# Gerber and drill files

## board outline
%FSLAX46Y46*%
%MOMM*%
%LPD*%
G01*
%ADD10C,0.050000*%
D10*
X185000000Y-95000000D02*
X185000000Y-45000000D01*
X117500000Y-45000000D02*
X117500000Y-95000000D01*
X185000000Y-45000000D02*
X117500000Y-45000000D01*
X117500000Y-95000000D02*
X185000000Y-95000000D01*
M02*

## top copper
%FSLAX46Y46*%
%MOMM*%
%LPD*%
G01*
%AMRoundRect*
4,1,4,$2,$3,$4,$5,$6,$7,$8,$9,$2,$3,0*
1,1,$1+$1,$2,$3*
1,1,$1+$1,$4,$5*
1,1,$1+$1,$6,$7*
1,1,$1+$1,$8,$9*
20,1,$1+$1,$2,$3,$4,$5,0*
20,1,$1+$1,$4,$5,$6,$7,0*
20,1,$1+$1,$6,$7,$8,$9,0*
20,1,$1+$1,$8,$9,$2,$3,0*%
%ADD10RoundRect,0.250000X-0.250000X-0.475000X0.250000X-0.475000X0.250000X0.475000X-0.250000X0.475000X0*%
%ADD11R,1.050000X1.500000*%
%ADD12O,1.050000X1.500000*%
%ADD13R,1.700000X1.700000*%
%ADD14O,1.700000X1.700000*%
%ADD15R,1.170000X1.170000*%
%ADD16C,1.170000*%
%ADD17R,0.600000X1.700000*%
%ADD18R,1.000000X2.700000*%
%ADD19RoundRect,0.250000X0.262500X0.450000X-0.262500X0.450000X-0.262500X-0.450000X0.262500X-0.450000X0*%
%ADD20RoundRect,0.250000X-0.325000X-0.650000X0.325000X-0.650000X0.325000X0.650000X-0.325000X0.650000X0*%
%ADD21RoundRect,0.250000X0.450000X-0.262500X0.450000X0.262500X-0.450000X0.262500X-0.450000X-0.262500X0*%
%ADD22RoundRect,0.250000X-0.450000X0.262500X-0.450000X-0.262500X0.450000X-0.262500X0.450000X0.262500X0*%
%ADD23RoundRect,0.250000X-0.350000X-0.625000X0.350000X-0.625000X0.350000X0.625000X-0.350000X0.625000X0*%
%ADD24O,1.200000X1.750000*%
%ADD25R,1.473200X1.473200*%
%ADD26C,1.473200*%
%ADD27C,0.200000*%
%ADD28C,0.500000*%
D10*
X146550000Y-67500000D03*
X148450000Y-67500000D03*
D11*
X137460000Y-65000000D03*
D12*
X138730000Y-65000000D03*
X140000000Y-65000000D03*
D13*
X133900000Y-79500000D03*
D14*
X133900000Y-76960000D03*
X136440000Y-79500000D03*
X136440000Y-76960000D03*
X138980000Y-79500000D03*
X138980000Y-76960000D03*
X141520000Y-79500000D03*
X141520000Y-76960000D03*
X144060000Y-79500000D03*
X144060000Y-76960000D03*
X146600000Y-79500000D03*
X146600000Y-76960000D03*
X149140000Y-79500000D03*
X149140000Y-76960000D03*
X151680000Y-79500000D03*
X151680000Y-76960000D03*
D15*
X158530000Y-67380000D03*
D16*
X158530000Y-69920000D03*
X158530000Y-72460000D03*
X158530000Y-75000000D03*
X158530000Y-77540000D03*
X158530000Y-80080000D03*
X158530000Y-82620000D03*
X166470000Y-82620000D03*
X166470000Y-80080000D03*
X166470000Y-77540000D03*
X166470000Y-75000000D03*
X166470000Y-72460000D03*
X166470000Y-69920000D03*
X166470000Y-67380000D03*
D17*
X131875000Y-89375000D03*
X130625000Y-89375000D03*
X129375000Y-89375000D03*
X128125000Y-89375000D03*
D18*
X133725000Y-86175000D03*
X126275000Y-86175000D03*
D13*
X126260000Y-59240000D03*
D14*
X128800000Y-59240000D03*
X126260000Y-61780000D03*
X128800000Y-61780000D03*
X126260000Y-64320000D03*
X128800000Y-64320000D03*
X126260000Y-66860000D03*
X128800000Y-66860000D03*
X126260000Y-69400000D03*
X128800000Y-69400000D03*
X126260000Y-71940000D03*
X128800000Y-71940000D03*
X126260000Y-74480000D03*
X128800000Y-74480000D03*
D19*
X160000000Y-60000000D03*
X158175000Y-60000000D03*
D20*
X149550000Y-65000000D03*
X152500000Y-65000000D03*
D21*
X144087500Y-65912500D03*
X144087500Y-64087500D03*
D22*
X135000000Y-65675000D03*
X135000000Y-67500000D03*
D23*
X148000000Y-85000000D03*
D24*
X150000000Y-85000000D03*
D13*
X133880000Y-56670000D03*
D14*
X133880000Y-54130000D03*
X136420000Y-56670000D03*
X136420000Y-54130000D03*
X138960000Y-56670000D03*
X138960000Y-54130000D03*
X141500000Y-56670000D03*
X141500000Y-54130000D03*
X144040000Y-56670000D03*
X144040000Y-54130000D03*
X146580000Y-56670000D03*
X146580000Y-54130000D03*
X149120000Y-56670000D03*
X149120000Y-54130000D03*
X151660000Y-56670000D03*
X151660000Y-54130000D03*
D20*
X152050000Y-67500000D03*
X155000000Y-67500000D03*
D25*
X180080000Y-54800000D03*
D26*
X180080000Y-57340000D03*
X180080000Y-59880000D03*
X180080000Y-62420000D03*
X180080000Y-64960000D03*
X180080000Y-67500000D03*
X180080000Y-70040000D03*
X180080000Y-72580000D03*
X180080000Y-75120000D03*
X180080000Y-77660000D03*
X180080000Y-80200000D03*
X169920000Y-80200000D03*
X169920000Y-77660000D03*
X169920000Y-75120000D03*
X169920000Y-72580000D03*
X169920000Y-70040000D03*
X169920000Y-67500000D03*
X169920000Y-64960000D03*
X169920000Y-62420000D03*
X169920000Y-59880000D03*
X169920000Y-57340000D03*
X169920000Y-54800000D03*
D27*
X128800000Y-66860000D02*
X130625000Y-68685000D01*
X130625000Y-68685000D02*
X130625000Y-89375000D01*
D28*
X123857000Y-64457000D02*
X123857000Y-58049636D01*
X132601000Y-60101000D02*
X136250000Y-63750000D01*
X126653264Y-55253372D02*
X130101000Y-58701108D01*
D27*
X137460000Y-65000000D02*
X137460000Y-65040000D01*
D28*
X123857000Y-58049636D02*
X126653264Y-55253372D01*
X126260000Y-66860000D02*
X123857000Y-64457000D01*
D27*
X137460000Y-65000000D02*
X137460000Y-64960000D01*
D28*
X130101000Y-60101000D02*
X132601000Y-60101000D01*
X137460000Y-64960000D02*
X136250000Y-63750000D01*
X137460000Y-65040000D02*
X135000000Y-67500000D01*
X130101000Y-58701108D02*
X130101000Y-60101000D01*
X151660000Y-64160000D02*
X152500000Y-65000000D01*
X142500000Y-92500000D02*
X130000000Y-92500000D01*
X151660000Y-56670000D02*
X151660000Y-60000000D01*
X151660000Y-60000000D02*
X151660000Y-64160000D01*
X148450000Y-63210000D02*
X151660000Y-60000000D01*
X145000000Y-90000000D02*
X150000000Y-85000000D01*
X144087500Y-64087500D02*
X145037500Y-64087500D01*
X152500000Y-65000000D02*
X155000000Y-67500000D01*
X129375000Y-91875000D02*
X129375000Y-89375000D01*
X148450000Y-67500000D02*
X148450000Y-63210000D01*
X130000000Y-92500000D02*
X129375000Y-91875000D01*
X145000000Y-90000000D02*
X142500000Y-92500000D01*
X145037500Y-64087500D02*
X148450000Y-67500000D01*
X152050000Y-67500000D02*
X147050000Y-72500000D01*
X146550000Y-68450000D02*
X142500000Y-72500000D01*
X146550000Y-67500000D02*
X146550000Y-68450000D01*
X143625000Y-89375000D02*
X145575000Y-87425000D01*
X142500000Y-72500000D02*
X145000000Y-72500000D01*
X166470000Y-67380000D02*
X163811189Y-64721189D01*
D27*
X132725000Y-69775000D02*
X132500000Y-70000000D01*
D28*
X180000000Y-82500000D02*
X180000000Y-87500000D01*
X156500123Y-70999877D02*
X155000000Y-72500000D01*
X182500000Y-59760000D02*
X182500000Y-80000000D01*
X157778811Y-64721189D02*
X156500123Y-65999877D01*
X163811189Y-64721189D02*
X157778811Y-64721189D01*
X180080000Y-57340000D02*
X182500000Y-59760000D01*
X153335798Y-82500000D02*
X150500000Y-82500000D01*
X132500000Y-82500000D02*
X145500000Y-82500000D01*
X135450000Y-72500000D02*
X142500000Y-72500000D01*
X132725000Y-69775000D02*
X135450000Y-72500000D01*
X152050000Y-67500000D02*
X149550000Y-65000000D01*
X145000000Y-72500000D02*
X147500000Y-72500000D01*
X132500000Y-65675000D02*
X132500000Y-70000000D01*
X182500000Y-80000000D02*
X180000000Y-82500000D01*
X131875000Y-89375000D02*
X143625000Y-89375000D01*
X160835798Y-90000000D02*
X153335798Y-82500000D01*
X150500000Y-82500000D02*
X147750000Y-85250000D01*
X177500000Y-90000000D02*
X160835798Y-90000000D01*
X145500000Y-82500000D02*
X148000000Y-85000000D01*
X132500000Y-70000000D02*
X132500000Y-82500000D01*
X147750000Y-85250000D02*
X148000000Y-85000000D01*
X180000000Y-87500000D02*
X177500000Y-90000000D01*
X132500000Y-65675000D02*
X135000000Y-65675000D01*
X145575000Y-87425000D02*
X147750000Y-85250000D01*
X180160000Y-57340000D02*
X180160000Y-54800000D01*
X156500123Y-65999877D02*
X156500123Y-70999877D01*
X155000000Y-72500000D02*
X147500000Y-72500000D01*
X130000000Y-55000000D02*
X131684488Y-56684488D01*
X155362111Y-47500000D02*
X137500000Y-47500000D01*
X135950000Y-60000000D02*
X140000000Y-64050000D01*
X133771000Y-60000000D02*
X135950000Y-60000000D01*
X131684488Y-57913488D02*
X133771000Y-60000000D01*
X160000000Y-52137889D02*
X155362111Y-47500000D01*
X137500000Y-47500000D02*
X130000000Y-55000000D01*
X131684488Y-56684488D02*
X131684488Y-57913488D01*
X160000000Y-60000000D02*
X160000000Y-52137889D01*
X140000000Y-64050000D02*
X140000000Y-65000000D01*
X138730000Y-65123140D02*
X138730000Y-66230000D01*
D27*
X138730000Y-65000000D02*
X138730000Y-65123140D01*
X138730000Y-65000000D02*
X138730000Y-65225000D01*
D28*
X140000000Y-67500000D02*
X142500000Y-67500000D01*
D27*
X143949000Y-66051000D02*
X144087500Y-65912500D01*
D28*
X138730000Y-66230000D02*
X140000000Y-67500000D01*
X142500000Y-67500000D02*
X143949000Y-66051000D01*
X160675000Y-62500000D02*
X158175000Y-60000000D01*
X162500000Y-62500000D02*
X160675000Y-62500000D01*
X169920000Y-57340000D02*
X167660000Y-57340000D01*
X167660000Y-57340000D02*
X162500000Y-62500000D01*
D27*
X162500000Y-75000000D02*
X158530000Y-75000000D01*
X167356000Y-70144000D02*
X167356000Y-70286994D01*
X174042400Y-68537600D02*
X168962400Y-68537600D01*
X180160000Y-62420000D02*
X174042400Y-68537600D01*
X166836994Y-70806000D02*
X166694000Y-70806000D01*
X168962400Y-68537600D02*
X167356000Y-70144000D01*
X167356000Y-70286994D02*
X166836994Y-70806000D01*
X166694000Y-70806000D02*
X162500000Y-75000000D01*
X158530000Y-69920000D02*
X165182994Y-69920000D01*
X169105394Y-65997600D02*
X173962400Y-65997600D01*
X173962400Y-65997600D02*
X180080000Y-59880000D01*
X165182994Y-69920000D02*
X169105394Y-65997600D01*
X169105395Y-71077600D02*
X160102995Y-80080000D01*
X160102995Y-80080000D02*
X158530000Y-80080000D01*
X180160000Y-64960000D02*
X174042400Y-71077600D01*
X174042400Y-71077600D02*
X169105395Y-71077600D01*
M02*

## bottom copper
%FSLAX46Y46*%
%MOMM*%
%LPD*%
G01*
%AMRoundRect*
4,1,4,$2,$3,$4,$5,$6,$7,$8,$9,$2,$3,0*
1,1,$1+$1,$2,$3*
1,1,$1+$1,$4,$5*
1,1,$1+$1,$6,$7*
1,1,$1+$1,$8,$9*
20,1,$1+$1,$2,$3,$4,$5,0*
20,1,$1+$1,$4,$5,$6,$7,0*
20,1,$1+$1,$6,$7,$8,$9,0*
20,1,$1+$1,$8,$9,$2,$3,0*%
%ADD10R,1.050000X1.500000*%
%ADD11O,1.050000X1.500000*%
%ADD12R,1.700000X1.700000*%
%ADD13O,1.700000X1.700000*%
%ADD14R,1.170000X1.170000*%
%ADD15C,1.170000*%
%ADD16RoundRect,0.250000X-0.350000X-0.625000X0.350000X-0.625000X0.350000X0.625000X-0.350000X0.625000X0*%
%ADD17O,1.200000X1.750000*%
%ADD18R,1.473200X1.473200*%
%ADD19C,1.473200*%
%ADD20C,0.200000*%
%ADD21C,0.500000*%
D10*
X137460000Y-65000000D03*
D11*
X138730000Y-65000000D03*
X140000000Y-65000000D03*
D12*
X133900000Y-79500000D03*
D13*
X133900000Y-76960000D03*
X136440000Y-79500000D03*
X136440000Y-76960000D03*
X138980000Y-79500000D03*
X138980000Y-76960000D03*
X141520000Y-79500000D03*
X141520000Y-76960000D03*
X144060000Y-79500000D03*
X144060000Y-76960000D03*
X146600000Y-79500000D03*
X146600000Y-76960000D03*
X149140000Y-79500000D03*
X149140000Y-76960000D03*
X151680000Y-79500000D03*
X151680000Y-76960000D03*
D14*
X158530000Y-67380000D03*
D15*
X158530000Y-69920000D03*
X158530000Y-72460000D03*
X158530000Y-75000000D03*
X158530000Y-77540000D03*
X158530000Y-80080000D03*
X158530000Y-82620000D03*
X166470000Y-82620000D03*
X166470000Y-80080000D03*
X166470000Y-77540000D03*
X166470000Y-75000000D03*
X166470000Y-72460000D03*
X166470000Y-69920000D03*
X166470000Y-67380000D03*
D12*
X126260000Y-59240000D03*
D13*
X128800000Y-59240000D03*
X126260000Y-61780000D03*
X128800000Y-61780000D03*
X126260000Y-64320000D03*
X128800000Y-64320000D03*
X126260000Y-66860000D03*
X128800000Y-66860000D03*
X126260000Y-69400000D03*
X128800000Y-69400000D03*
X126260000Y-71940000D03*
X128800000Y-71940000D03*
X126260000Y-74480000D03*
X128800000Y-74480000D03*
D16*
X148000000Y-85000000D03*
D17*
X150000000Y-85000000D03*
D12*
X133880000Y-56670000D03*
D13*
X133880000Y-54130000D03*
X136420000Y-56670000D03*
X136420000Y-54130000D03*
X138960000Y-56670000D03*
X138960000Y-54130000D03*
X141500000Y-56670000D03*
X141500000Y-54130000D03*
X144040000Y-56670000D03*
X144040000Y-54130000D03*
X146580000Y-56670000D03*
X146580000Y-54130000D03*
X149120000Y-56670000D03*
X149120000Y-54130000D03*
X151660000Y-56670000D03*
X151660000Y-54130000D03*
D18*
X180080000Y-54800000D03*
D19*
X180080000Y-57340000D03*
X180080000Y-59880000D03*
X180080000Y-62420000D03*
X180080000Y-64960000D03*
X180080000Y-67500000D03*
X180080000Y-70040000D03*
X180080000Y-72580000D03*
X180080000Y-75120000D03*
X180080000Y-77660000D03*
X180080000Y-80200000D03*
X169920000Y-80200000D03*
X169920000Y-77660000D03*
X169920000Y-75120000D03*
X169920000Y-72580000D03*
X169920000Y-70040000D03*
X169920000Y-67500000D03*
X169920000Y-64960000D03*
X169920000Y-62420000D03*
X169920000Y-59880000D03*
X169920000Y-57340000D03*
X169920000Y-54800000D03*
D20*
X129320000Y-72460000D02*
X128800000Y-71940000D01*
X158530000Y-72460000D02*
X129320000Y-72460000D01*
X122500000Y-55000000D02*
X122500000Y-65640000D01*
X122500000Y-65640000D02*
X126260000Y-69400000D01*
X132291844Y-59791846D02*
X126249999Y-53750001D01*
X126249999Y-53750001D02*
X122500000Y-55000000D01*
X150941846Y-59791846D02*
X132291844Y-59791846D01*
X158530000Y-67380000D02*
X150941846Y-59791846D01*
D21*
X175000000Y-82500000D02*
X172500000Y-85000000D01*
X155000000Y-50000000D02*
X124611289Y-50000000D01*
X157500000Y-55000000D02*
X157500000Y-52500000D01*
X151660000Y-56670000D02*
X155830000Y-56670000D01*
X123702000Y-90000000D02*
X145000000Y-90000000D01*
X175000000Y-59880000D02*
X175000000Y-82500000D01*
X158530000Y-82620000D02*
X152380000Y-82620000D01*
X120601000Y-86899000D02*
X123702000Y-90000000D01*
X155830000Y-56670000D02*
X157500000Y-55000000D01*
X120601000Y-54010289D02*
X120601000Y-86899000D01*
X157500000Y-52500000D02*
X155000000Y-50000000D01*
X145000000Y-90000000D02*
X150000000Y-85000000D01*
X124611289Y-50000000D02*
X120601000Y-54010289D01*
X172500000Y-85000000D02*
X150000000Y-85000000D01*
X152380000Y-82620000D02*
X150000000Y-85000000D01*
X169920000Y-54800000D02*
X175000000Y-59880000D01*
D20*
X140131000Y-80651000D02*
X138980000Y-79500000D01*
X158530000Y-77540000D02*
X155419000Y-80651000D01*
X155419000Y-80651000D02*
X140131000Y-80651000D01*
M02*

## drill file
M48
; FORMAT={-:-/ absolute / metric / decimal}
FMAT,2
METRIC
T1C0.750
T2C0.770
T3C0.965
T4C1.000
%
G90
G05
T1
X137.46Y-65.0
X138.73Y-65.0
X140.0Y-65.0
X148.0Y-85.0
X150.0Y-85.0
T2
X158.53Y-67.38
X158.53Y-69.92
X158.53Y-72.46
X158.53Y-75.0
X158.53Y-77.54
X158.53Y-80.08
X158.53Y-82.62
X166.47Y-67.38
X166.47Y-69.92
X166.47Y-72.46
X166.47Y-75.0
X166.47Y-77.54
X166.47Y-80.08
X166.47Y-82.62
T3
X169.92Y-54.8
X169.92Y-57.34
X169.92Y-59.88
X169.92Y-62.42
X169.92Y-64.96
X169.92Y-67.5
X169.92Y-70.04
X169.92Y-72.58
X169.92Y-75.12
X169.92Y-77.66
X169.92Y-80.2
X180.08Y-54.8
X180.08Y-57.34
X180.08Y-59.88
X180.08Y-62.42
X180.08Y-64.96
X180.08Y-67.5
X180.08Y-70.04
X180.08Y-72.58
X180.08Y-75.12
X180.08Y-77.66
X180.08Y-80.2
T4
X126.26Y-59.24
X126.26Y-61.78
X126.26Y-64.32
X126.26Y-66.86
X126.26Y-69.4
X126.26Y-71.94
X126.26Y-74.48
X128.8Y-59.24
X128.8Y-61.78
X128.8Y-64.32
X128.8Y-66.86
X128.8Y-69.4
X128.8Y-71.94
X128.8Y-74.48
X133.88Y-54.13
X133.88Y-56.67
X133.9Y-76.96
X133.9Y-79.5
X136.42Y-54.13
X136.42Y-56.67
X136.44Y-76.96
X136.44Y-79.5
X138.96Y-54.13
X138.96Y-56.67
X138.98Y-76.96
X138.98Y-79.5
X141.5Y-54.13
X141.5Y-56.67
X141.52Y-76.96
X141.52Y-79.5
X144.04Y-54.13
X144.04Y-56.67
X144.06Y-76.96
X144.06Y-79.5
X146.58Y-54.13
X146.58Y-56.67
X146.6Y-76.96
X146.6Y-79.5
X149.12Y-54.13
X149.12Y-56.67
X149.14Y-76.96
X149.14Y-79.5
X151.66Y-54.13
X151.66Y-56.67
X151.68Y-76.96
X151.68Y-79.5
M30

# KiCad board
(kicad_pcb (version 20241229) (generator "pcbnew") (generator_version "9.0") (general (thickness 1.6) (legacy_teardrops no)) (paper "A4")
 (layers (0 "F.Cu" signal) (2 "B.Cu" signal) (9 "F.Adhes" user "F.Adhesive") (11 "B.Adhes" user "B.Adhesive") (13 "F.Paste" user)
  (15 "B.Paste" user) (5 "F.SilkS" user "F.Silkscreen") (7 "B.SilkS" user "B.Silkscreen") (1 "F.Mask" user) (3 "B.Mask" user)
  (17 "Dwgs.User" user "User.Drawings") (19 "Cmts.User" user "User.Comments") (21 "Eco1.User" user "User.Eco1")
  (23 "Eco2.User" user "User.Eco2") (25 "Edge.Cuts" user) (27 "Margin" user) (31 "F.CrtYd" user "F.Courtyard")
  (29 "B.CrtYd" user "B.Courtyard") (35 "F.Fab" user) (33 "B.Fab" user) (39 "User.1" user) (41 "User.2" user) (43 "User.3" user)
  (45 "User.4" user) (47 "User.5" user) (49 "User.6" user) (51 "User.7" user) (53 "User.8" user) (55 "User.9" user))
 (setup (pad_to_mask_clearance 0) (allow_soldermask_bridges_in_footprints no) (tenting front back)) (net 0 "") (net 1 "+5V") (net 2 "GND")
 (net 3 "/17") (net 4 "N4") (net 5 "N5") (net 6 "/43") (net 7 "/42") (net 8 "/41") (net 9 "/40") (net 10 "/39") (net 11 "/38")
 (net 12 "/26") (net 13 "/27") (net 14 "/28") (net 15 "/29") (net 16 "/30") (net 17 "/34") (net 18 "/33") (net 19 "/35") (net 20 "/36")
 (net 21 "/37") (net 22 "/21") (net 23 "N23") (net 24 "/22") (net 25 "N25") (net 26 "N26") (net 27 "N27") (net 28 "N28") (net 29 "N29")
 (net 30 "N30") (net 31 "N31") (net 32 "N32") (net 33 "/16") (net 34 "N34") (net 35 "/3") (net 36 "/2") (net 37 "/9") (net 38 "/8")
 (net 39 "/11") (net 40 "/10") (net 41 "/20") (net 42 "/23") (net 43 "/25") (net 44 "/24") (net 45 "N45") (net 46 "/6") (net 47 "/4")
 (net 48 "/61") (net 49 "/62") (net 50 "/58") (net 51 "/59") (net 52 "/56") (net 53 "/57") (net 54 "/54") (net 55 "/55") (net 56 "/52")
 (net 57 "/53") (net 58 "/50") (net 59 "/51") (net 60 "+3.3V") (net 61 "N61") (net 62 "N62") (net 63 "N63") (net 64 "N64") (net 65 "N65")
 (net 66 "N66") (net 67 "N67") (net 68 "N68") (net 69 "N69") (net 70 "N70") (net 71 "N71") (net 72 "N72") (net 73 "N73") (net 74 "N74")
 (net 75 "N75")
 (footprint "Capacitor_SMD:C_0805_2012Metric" (layer "F.Cu") (at 147.5 67.5)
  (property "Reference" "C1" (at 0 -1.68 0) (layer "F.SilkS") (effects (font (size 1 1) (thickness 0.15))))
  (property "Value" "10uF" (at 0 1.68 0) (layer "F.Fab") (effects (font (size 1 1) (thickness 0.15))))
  (pad "1" smd roundrect (at -0.95 0) (size 1 1.45) (layers "F.Cu" "F.Mask" "F.Paste") (roundrect_rratio 0.25) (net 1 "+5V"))
  (pad "2" smd roundrect (at 0.95 0) (size 1 1.45) (layers "F.Cu" "F.Mask" "F.Paste") (roundrect_rratio 0.25) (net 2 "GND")))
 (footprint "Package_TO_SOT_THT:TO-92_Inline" (layer "F.Cu") (at 137.46 65)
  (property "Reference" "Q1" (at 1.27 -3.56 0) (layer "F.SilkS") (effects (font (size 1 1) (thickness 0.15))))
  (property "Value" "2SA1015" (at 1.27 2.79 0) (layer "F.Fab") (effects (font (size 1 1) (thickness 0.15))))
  (pad "1" thru_hole rect (at 0 0) (size 1.05 1.5) (drill 0.75) (layers "*.Cu" "*.Mask") (remove_unused_layers no) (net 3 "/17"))
  (pad "2" thru_hole oval (at 1.27 0) (size 1.05 1.5) (drill 0.75) (layers "*.Cu" "*.Mask") (remove_unused_layers no) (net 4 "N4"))
  (pad "3" thru_hole oval (at 2.54 0) (size 1.05 1.5) (drill 0.75) (layers "*.Cu" "*.Mask") (remove_unused_layers no) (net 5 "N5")))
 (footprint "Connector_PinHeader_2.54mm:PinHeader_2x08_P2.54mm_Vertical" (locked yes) (layer "F.Cu") (at 133.9 79.5 90)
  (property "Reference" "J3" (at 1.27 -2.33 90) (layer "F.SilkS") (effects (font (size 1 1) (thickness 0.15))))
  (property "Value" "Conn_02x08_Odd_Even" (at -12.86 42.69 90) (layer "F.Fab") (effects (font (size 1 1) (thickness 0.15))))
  (pad "1" thru_hole rect (at 0 0 90) (size 1.7 1.7) (drill 1) (layers "*.Cu" "*.Mask") (remove_unused_layers no) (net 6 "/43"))
  (pad "2" thru_hole oval (at 2.54 0 90) (size 1.7 1.7) (drill 1) (layers "*.Cu" "*.Mask") (remove_unused_layers no) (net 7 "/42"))
  (pad "3" thru_hole oval (at 0 2.54 90) (size 1.7 1.7) (drill 1) (layers "*.Cu" "*.Mask") (remove_unused_layers no) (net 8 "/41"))
  (pad "4" thru_hole oval (at 2.54 2.54 90) (size 1.7 1.7) (drill 1) (layers "*.Cu" "*.Mask") (remove_unused_layers no) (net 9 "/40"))
  (pad "5" thru_hole oval (at 0 5.08 90) (size 1.7 1.7) (drill 1) (layers "*.Cu" "*.Mask") (remove_unused_layers no) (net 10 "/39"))
  (pad "6" thru_hole oval (at 2.54 5.08 90) (size 1.7 1.7) (drill 1) (layers "*.Cu" "*.Mask") (remove_unused_layers no) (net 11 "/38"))
  (pad "7" thru_hole oval (at 0 7.62 90) (size 1.7 1.7) (drill 1) (layers "*.Cu" "*.Mask") (remove_unused_layers no) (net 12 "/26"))
  (pad "8" thru_hole oval (at 2.54 7.62 90) (size 1.7 1.7) (drill 1) (layers "*.Cu" "*.Mask") (remove_unused_layers no) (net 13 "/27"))
  (pad "9" thru_hole oval (at 0 10.16 90) (size 1.7 1.7) (drill 1) (layers "*.Cu" "*.Mask") (remove_unused_layers no) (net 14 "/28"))
  (pad "10" thru_hole oval (at 2.54 10.16 90) (size 1.7 1.7) (drill 1) (layers "*.Cu" "*.Mask") (remove_unused_layers no) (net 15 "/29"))
  (pad "11" thru_hole oval (at 0 12.7 90) (size 1.7 1.7) (drill 1) (layers "*.Cu" "*.Mask") (remove_unused_layers no) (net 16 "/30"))
  (pad "12" thru_hole oval (at 2.54 12.7 90) (size 1.7 1.7) (drill 1) (layers "*.Cu" "*.Mask") (remove_unused_layers no) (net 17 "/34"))
  (pad "13" thru_hole oval (at 0 15.24 90) (size 1.7 1.7) (drill 1) (layers "*.Cu" "*.Mask") (remove_unused_layers no) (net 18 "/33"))
  (pad "14" thru_hole oval (at 2.54 15.24 90) (size 1.7 1.7) (drill 1) (layers "*.Cu" "*.Mask") (remove_unused_layers no) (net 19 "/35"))
  (pad "15" thru_hole oval (at 0 17.78 90) (size 1.7 1.7) (drill 1) (layers "*.Cu" "*.Mask") (remove_unused_layers no) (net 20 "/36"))
  (pad "16" thru_hole oval (at 2.54 17.78 90) (size 1.7 1.7) (drill 1) (layers "*.Cu" "*.Mask") (remove_unused_layers no) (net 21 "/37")))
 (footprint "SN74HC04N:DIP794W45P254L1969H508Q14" (layer "F.Cu") (at 162.5 75)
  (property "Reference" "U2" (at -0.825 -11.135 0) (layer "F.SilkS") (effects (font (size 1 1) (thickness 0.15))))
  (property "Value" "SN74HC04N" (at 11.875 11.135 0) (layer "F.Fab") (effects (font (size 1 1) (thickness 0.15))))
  (pad "1" thru_hole rect (at -3.97 -7.62) (size 1.17 1.17) (drill 0.77) (layers "*.Cu" "*.Mask") (remove_unused_layers no) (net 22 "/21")
   (solder_mask_margin 0.102))
  (pad "2" thru_hole circle (at -3.97 -5.08) (size 1.17 1.17) (drill 0.77) (layers "*.Cu" "*.Mask") (remove_unused_layers no) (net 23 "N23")
   (solder_mask_margin 0.102))
  (pad "3" thru_hole circle (at -3.97 -2.54) (size 1.17 1.17) (drill 0.77) (layers "*.Cu" "*.Mask") (remove_unused_layers no) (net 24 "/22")
   (solder_mask_margin 0.102))
  (pad "4" thru_hole circle (at -3.97 0) (size 1.17 1.17) (drill 0.77) (layers "*.Cu" "*.Mask") (remove_unused_layers no) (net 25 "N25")
   (solder_mask_margin 0.102))
  (pad "5" thru_hole circle (at -3.97 2.54) (size 1.17 1.17) (drill 0.77) (layers "*.Cu" "*.Mask") (remove_unused_layers no) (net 10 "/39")
   (solder_mask_margin 0.102))
  (pad "6" thru_hole circle (at -3.97 5.08) (size 1.17 1.17) (drill 0.77) (layers "*.Cu" "*.Mask") (remove_unused_layers no) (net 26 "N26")
   (solder_mask_margin 0.102))
  (pad "7" thru_hole circle (at -3.97 7.62) (size 1.17 1.17) (drill 0.77) (layers "*.Cu" "*.Mask") (remove_unused_layers no) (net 2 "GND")
   (solder_mask_margin 0.102))
  (pad "8" thru_hole circle (at 3.97 7.62) (size 1.17 1.17) (drill 0.77) (layers "*.Cu" "*.Mask") (remove_unused_layers no) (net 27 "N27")
   (solder_mask_margin 0.102))
  (pad "9" thru_hole circle (at 3.97 5.08) (size 1.17 1.17) (drill 0.77) (layers "*.Cu" "*.Mask") (remove_unused_layers no) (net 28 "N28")
   (solder_mask_margin 0.102))
  (pad "10" thru_hole circle (at 3.97 2.54) (size 1.17 1.17) (drill 0.77) (layers "*.Cu" "*.Mask") (remove_unused_layers no) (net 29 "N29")
   (solder_mask_margin 0.102))
  (pad "11" thru_hole circle (at 3.97 0) (size 1.17 1.17) (drill 0.77) (layers "*.Cu" "*.Mask") (remove_unused_layers no) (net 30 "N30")
   (solder_mask_margin 0.102))
  (pad "12" thru_hole circle (at 3.97 -2.54) (size 1.17 1.17) (drill 0.77) (layers "*.Cu" "*.Mask") (remove_unused_layers no) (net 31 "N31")
   (solder_mask_margin 0.102))
  (pad "13" thru_hole circle (at 3.97 -5.08) (size 1.17 1.17) (drill 0.77) (layers "*.Cu" "*.Mask") (remove_unused_layers no) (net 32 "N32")
   (solder_mask_margin 0.102))
  (pad "14" thru_hole circle (at 3.97 -7.62) (size 1.17 1.17) (drill 0.77) (layers "*.Cu" "*.Mask") (remove_unused_layers no) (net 1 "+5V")
   (solder_mask_margin 0.102)))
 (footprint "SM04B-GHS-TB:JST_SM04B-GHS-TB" (layer "F.Cu") (at 130 87.5 180)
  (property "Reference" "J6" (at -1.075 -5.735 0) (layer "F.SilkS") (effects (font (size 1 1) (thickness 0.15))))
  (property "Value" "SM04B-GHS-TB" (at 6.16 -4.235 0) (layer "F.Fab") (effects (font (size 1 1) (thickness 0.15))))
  (pad "1" smd rect (at -1.875 -1.875 180) (size 0.6 1.7) (layers "F.Cu" "F.Mask" "F.Paste") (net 1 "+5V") (solder_mask_margin 0.102))
  (pad "2" smd rect (at -0.625 -1.875 180) (size 0.6 1.7) (layers "F.Cu" "F.Mask" "F.Paste") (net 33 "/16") (solder_mask_margin 0.102))
  (pad "3" smd rect (at 0.625 -1.875 180) (size 0.6 1.7) (layers "F.Cu" "F.Mask" "F.Paste") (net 2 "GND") (solder_mask_margin 0.102))
  (pad "4" smd rect (at 1.875 -1.875 180) (size 0.6 1.7) (layers "F.Cu" "F.Mask" "F.Paste") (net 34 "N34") (solder_mask_margin 0.102))
  (pad "MP1" smd rect (at -3.725 1.325 180) (size 1 2.7) (layers "F.Cu" "F.Mask" "F.Paste") (solder_mask_margin 0.102))
  (pad "MP2" smd rect (at 3.725 1.325 180) (size 1 2.7) (layers "F.Cu" "F.Mask" "F.Paste") (solder_mask_margin 0.102)))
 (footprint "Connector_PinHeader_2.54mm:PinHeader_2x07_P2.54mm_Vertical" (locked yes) (layer "F.Cu") (at 126.26 59.24)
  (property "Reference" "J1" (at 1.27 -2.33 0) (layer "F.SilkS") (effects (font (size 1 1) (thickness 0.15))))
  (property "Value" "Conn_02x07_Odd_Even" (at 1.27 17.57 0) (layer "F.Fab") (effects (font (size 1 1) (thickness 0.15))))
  (pad "1" thru_hole rect (at 0 0) (size 1.7 1.7) (drill 1) (layers "*.Cu" "*.Mask") (remove_unused_layers no) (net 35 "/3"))
  (pad "2" thru_hole oval (at 2.54 0) (size 1.7 1.7) (drill 1) (layers "*.Cu" "*.Mask") (remove_unused_layers no) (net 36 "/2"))
  (pad "3" thru_hole oval (at 0 2.54) (size 1.7 1.7) (drill 1) (layers "*.Cu" "*.Mask") (remove_unused_layers no) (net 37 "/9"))
  (pad "4" thru_hole oval (at 2.54 2.54) (size 1.7 1.7) (drill 1) (layers "*.Cu" "*.Mask") (remove_unused_layers no) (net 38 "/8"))
  (pad "5" thru_hole oval (at 0 5.08) (size 1.7 1.7) (drill 1) (layers "*.Cu" "*.Mask") (remove_unused_layers no) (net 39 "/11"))
  (pad "6" thru_hole oval (at 2.54 5.08) (size 1.7 1.7) (drill 1) (layers "*.Cu" "*.Mask") (remove_unused_layers no) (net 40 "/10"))
  (pad "7" thru_hole oval (at 0 7.62) (size 1.7 1.7) (drill 1) (layers "*.Cu" "*.Mask") (remove_unused_layers no) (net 3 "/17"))
  (pad "8" thru_hole oval (at 2.54 7.62) (size 1.7 1.7) (drill 1) (layers "*.Cu" "*.Mask") (remove_unused_layers no) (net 33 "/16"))
  (pad "9" thru_hole oval (at 0 10.16) (size 1.7 1.7) (drill 1) (layers "*.Cu" "*.Mask") (remove_unused_layers no) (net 22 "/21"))
  (pad "10" thru_hole oval (at 2.54 10.16) (size 1.7 1.7) (drill 1) (layers "*.Cu" "*.Mask") (remove_unused_layers no) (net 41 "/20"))
  (pad "11" thru_hole oval (at 0 12.7) (size 1.7 1.7) (drill 1) (layers "*.Cu" "*.Mask") (remove_unused_layers no) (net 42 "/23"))
  (pad "12" thru_hole oval (at 2.54 12.7) (size 1.7 1.7) (drill 1) (layers "*.Cu" "*.Mask") (remove_unused_layers no) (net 24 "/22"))
  (pad "13" thru_hole oval (at 0 15.24) (size 1.7 1.7) (drill 1) (layers "*.Cu" "*.Mask") (remove_unused_layers no) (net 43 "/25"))
  (pad "14" thru_hole oval (at 2.54 15.24) (size 1.7 1.7) (drill 1) (layers "*.Cu" "*.Mask") (remove_unused_layers no) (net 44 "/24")))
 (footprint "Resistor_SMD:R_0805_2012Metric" (layer "F.Cu") (at 159.0875 60 180)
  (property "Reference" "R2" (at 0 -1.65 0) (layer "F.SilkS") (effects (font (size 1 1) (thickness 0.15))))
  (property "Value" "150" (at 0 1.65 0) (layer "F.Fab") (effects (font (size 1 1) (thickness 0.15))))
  (pad "1" smd roundrect (at -0.9125 0 180) (size 1.025 1.4) (layers "F.Cu" "F.Mask" "F.Paste") (roundrect_rratio 0.243902) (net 5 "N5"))
  (pad "2" smd roundrect (at 0.9125 0 180) (size 1.025 1.4) (layers "F.Cu" "F.Mask" "F.Paste") (roundrect_rratio 0.243902) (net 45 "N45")))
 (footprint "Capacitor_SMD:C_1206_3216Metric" (layer "F.Cu") (at 151.025 65)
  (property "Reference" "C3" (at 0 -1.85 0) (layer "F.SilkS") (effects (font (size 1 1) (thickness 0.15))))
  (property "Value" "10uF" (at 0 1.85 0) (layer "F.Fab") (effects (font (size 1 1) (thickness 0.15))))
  (pad "1" smd roundrect (at -1.475 0) (size 1.15 1.8) (layers "F.Cu" "F.Mask" "F.Paste") (roundrect_rratio 0.217391) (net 1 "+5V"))
  (pad "2" smd roundrect (at 1.475 0) (size 1.15 1.8) (layers "F.Cu" "F.Mask" "F.Paste") (roundrect_rratio 0.217391) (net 2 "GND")))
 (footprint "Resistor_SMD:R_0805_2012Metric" (layer "F.Cu") (at 144.0875 65 90)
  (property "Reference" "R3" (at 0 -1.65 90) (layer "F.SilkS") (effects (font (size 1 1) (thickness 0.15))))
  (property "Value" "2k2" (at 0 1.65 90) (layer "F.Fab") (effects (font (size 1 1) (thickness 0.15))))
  (pad "1" smd roundrect (at -0.9125 0 90) (size 1.025 1.4) (layers "F.Cu" "F.Mask" "F.Paste") (roundrect_rratio 0.243902) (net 4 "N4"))
  (pad "2" smd roundrect (at 0.9125 0 90) (size 1.025 1.4) (layers "F.Cu" "F.Mask" "F.Paste") (roundrect_rratio 0.243902) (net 2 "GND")))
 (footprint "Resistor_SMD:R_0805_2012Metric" (layer "F.Cu") (at 135 66.5875 -90)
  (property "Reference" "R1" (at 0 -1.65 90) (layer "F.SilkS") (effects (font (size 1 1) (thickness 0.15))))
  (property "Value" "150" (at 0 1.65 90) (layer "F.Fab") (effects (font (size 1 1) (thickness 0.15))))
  (pad "1" smd roundrect (at -0.9125 0 270) (size 1.025 1.4) (layers "F.Cu" "F.Mask" "F.Paste") (roundrect_rratio 0.243902) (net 1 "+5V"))
  (pad "2" smd roundrect (at 0.9125 0 270) (size 1.025 1.4) (layers "F.Cu" "F.Mask" "F.Paste") (roundrect_rratio 0.243902) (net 3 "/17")))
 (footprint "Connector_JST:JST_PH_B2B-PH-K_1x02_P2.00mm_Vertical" (layer "F.Cu") (at 148 85)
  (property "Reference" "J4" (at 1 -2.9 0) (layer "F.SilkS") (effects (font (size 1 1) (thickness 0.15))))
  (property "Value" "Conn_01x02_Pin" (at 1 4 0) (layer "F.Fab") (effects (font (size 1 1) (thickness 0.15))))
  (pad "1" thru_hole roundrect (at 0 0) (size 1.2 1.75) (drill 0.75) (layers "*.Cu" "*.Mask") (remove_unused_layers no)
   (roundrect_rratio 0.208333) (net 1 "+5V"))
  (pad "2" thru_hole oval (at 2 0) (size 1.2 1.75) (drill 0.75) (layers "*.Cu" "*.Mask") (remove_unused_layers no) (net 2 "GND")))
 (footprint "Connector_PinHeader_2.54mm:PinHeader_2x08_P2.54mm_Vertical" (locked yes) (layer "F.Cu") (at 133.88 56.67 90)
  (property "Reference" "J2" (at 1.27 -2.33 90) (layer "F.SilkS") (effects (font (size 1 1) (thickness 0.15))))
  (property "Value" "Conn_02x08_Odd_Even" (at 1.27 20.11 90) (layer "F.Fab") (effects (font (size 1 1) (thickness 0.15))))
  (pad "1" thru_hole rect (at 0 0 90) (size 1.7 1.7) (drill 1) (layers "*.Cu" "*.Mask") (remove_unused_layers no) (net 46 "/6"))
  (pad "2" thru_hole oval (at 2.54 0 90) (size 1.7 1.7) (drill 1) (layers "*.Cu" "*.Mask") (remove_unused_layers no) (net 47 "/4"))
  (pad "3" thru_hole oval (at 0 2.54 90) (size 1.7 1.7) (drill 1) (layers "*.Cu" "*.Mask") (remove_unused_layers no) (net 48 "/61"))
  (pad "4" thru_hole oval (at 2.54 2.54 90) (size 1.7 1.7) (drill 1) (layers "*.Cu" "*.Mask") (remove_unused_layers no) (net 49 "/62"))
  (pad "5" thru_hole oval (at 0 5.08 90) (size 1.7 1.7) (drill 1) (layers "*.Cu" "*.Mask") (remove_unused_layers no) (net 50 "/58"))
  (pad "6" thru_hole oval (at 2.54 5.08 90) (size 1.7 1.7) (drill 1) (layers "*.Cu" "*.Mask") (remove_unused_layers no) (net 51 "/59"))
  (pad "7" thru_hole oval (at 0 7.62 90) (size 1.7 1.7) (drill 1) (layers "*.Cu" "*.Mask") (remove_unused_layers no) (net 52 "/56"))
  (pad "8" thru_hole oval (at 2.54 7.62 90) (size 1.7 1.7) (drill 1) (layers "*.Cu" "*.Mask") (remove_unused_layers no) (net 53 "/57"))
  (pad "9" thru_hole oval (at 0 10.16 90) (size 1.7 1.7) (drill 1) (layers "*.Cu" "*.Mask") (remove_unused_layers no) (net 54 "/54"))
  (pad "10" thru_hole oval (at 2.54 10.16 90) (size 1.7 1.7) (drill 1) (layers "*.Cu" "*.Mask") (remove_unused_layers no) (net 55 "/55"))
  (pad "11" thru_hole oval (at 0 12.7 90) (size 1.7 1.7) (drill 1) (layers "*.Cu" "*.Mask") (remove_unused_layers no) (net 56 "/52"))
  (pad "12" thru_hole oval (at 2.54 12.7 90) (size 1.7 1.7) (drill 1) (layers "*.Cu" "*.Mask") (remove_unused_layers no) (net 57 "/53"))
  (pad "13" thru_hole oval (at 0 15.24 90) (size 1.7 1.7) (drill 1) (layers "*.Cu" "*.Mask") (remove_unused_layers no) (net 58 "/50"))
  (pad "14" thru_hole oval (at 2.54 15.24 90) (size 1.7 1.7) (drill 1) (layers "*.Cu" "*.Mask") (remove_unused_layers no) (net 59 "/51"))
  (pad "15" thru_hole oval (at 0 17.78 90) (size 1.7 1.7) (drill 1) (layers "*.Cu" "*.Mask") (remove_unused_layers no) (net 2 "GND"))
  (pad "16" thru_hole oval (at 2.54 17.78 90) (size 1.7 1.7) (drill 1) (layers "*.Cu" "*.Mask") (remove_unused_layers no) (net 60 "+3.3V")))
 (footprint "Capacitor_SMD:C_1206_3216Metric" (layer "F.Cu") (at 153.525 67.5)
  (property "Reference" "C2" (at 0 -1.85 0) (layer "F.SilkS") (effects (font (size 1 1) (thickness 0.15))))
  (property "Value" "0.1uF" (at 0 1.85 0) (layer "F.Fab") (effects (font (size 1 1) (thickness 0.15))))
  (pad "1" smd roundrect (at -1.475 0) (size 1.15 1.8) (layers "F.Cu" "F.Mask" "F.Paste") (roundrect_rratio 0.217391) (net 1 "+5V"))
  (pad "2" smd roundrect (at 1.475 0) (size 1.15 1.8) (layers "F.Cu" "F.Mask" "F.Paste") (roundrect_rratio 0.217391) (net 2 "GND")))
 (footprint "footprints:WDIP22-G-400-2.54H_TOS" (layer "B.Cu") (at 180.08 54.8 180)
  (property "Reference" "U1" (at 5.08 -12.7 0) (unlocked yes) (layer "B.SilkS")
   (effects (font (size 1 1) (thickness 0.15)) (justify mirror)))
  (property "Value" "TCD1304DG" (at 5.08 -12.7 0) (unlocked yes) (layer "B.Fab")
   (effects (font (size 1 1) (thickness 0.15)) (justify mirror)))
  (pad "1" thru_hole rect (at 0 0 180) (size 1.4732 1.4732) (drill 0.9652) (layers "*.Cu" "*.Mask") (remove_unused_layers no) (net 1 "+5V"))
  (pad "2" thru_hole circle (at 0 -2.54 180) (size 1.4732 1.4732) (drill 0.9652) (layers "*.Cu" "*.Mask") (remove_unused_layers no)
   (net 1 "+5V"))
  (pad "3" thru_hole circle (at 0 -5.08 180) (size 1.4732 1.4732) (drill 0.9652) (layers "*.Cu" "*.Mask") (remove_unused_layers no)
   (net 23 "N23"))
  (pad "4" thru_hole circle (at 0 -7.62 180) (size 1.4732 1.4732) (drill 0.9652) (layers "*.Cu" "*.Mask") (remove_unused_layers no)
   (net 25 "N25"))
  (pad "5" thru_hole circle (at 0 -10.16 180) (size 1.4732 1.4732) (drill 0.9652) (layers "*.Cu" "*.Mask") (remove_unused_layers no)
   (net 26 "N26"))
  (pad "6" thru_hole circle (at 0 -12.7 180) (size 1.4732 1.4732) (drill 0.9652) (layers "*.Cu" "*.Mask") (remove_unused_layers no)
   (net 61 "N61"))
  (pad "7" thru_hole circle (at 0 -15.24 180) (size 1.4732 1.4732) (drill 0.9652) (layers "*.Cu" "*.Mask") (remove_unused_layers no)
   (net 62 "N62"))
  (pad "8" thru_hole circle (at 0 -17.78 180) (size 1.4732 1.4732) (drill 0.9652) (layers "*.Cu" "*.Mask") (remove_unused_layers no)
   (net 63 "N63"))
  (pad "9" thru_hole circle (at 0 -20.32 180) (size 1.4732 1.4732) (drill 0.9652) (layers "*.Cu" "*.Mask") (remove_unused_layers no)
   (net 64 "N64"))
  (pad "10" thru_hole circle (at 0 -22.86 180) (size 1.4732 1.4732) (drill 0.9652) (layers "*.Cu" "*.Mask") (remove_unused_layers no)
   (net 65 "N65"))
  (pad "11" thru_hole circle (at 0 -25.4 180) (size 1.4732 1.4732) (drill 0.9652) (layers "*.Cu" "*.Mask") (remove_unused_layers no)
   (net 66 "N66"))
  (pad "12" thru_hole circle (at 10.16 -25.4 180) (size 1.4732 1.4732) (drill 0.9652) (layers "*.Cu" "*.Mask") (remove_unused_layers no)
   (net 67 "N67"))
  (pad "13" thru_hole circle (at 10.16 -22.86 180) (size 1.4732 1.4732) (drill 0.9652) (layers "*.Cu" "*.Mask") (remove_unused_layers no)
   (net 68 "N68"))
  (pad "14" thru_hole circle (at 10.16 -20.32 180) (size 1.4732 1.4732) (drill 0.9652) (layers "*.Cu" "*.Mask") (remove_unused_layers no)
   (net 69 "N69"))
  (pad "15" thru_hole circle (at 10.16 -17.78 180) (size 1.4732 1.4732) (drill 0.9652) (layers "*.Cu" "*.Mask") (remove_unused_layers no)
   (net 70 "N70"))
  (pad "16" thru_hole circle (at 10.16 -15.24 180) (size 1.4732 1.4732) (drill 0.9652) (layers "*.Cu" "*.Mask") (remove_unused_layers no)
   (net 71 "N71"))
  (pad "17" thru_hole circle (at 10.16 -12.7 180) (size 1.4732 1.4732) (drill 0.9652) (layers "*.Cu" "*.Mask") (remove_unused_layers no)
   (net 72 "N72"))
  (pad "18" thru_hole circle (at 10.16 -10.16 180) (size 1.4732 1.4732) (drill 0.9652) (layers "*.Cu" "*.Mask") (remove_unused_layers no)
   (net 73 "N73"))
  (pad "19" thru_hole circle (at 10.16 -7.62 180) (size 1.4732 1.4732) (drill 0.9652) (layers "*.Cu" "*.Mask") (remove_unused_layers no)
   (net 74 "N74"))
  (pad "20" thru_hole circle (at 10.16 -5.08 180) (size 1.4732 1.4732) (drill 0.9652) (layers "*.Cu" "*.Mask") (remove_unused_layers no)
   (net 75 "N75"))
  (pad "21" thru_hole circle (at 10.16 -2.54 180) (size 1.4732 1.4732) (drill 0.9652) (layers "*.Cu" "*.Mask") (remove_unused_layers no)
   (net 45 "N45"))
  (pad "22" thru_hole circle (at 10.16 0 180) (size 1.4732 1.4732) (drill 0.9652) (layers "*.Cu" "*.Mask") (remove_unused_layers no)
   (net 2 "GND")))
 (gr_line (start 185 95) (end 185 45) (stroke (width 0.05) (type default)) (layer "Edge.Cuts"))
 (gr_line (start 117.5 45) (end 117.5 95) (stroke (width 0.05) (type default)) (layer "Edge.Cuts"))
 (gr_line (start 185 45) (end 117.5 45) (stroke (width 0.05) (type default)) (layer "Edge.Cuts"))
 (gr_line (start 117.5 95) (end 185 95) (stroke (width 0.05) (type default)) (layer "Edge.Cuts"))
 (segment (start 128.8 66.86) (end 130.625 68.685) (width 0.2) (layer "F.Cu") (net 33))
 (segment (start 130.625 68.685) (end 130.625 89.375) (width 0.2) (layer "F.Cu") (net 33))
 (segment (start 129.32 72.46) (end 128.8 71.94) (width 0.2) (layer "B.Cu") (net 24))
 (segment (start 158.53 72.46) (end 129.32 72.46) (width 0.2) (layer "B.Cu") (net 24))
 (segment (start 123.857 64.457) (end 123.857 58.049636) (width 0.5) (layer "F.Cu") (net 3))
 (segment (start 132.601 60.101) (end 136.25 63.75) (width 0.5) (layer "F.Cu") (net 3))
 (segment (start 126.653264 55.253372) (end 130.101 58.701108) (width 0.5) (layer "F.Cu") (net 3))
 (segment (start 137.46 65) (end 137.46 65.04) (width 0.2) (layer "F.Cu") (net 3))
 (segment (start 123.857 58.049636) (end 126.653264 55.253372) (width 0.5) (layer "F.Cu") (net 3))
 (segment (start 126.26 66.86) (end 123.857 64.457) (width 0.5) (layer "F.Cu") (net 3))
 (segment (start 137.46 65) (end 137.46 64.96) (width 0.2) (layer "F.Cu") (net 3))
 (segment (start 130.101 60.101) (end 132.601 60.101) (width 0.5) (layer "F.Cu") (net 3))
 (segment (start 137.46 64.96) (end 136.25 63.75) (width 0.5) (layer "F.Cu") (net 3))
 (segment (start 137.46 65.04) (end 135 67.5) (width 0.5) (layer "F.Cu") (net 3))
 (segment (start 130.101 58.701108) (end 130.101 60.101) (width 0.5) (layer "F.Cu") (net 3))
 (segment (start 122.5 55) (end 122.5 65.64) (width 0.2) (layer "B.Cu") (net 22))
 (segment (start 122.5 65.64) (end 126.26 69.4) (width 0.2) (layer "B.Cu") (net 22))
 (segment (start 132.291844 59.791846) (end 126.249999 53.750001) (width 0.2) (layer "B.Cu") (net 22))
 (segment (start 126.249999 53.750001) (end 122.5 55) (width 0.2) (layer "B.Cu") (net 22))
 (segment (start 150.941846 59.791846) (end 132.291844 59.791846) (width 0.2) (layer "B.Cu") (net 22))
 (segment (start 158.53 67.38) (end 150.941846 59.791846) (width 0.2) (layer "B.Cu") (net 22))
 (segment (start 151.66 64.16) (end 152.5 65) (width 0.5) (layer "F.Cu") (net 2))
 (segment (start 142.5 92.5) (end 130 92.5) (width 0.5) (layer "F.Cu") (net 2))
 (segment (start 151.66 56.67) (end 151.66 60) (width 0.5) (layer "F.Cu") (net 2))
 (segment (start 151.66 60) (end 151.66 64.16) (width 0.5) (layer "F.Cu") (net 2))
 (segment (start 148.45 63.21) (end 151.66 60) (width 0.5) (layer "F.Cu") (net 2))
 (segment (start 145 90) (end 150 85) (width 0.5) (layer "F.Cu") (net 2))
 (segment (start 144.0875 64.0875) (end 145.0375 64.0875) (width 0.5) (layer "F.Cu") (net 2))
 (segment (start 152.5 65) (end 155 67.5) (width 0.5) (layer "F.Cu") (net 2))
 (segment (start 129.375 91.875) (end 129.375 89.375) (width 0.5) (layer "F.Cu") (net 2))
 (segment (start 148.45 67.5) (end 148.45 63.21) (width 0.5) (layer "F.Cu") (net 2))
 (segment (start 130 92.5) (end 129.375 91.875) (width 0.5) (layer "F.Cu") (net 2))
 (segment (start 145 90) (end 142.5 92.5) (width 0.5) (layer "F.Cu") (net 2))
 (segment (start 145.0375 64.0875) (end 148.45 67.5) (width 0.5) (layer "F.Cu") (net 2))
 (segment (start 175 82.5) (end 172.5 85) (width 0.5) (layer "B.Cu") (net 2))
 (segment (start 155 50) (end 124.611289 50) (width 0.5) (layer "B.Cu") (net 2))
 (segment (start 157.5 55) (end 157.5 52.5) (width 0.5) (layer "B.Cu") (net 2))
 (segment (start 151.66 56.67) (end 155.83 56.67) (width 0.5) (layer "B.Cu") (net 2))
 (segment (start 123.702 90) (end 145 90) (width 0.5) (layer "B.Cu") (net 2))
 (segment (start 175 59.88) (end 175 82.5) (width 0.5) (layer "B.Cu") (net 2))
 (segment (start 158.53 82.62) (end 152.38 82.62) (width 0.5) (layer "B.Cu") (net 2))
 (segment (start 120.601 86.899) (end 123.702 90) (width 0.5) (layer "B.Cu") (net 2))
 (segment (start 155.83 56.67) (end 157.5 55) (width 0.5) (layer "B.Cu") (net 2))
 (segment (start 120.601 54.010289) (end 120.601 86.899) (width 0.5) (layer "B.Cu") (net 2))
 (segment (start 157.5 52.5) (end 155 50) (width 0.5) (layer "B.Cu") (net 2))
 (segment (start 145 90) (end 150 85) (width 0.5) (layer "B.Cu") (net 2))
 (segment (start 124.611289 50) (end 120.601 54.010289) (width 0.5) (layer "B.Cu") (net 2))
 (segment (start 172.5 85) (end 150 85) (width 0.5) (layer "B.Cu") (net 2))
 (segment (start 152.38 82.62) (end 150 85) (width 0.5) (layer "B.Cu") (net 2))
 (segment (start 169.92 54.8) (end 175 59.88) (width 0.5) (layer "B.Cu") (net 2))
 (segment (start 140.131 80.651) (end 138.98 79.5) (width 0.2) (layer "B.Cu") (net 10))
 (segment (start 158.53 77.54) (end 155.419 80.651) (width 0.2) (layer "B.Cu") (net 10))
 (segment (start 155.419 80.651) (end 140.131 80.651) (width 0.2) (layer "B.Cu") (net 10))
 (segment (start 152.05 67.5) (end 147.05 72.5) (width 0.5) (layer "F.Cu") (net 1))
 (segment (start 146.55 68.45) (end 142.5 72.5) (width 0.5) (layer "F.Cu") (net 1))
 (segment (start 146.55 67.5) (end 146.55 68.45) (width 0.5) (layer "F.Cu") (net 1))
 (segment (start 143.625 89.375) (end 145.575 87.425) (width 0.5) (layer "F.Cu") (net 1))
 (segment (start 142.5 72.5) (end 145 72.5) (width 0.5) (layer "F.Cu") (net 1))
 (segment (start 166.47 67.38) (end 163.811189 64.721189) (width 0.5) (layer "F.Cu") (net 1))
 (segment (start 132.725 69.775) (end 132.5 70) (width 0.2) (layer "F.Cu") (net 1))
 (segment (start 180 82.5) (end 180 87.5) (width 0.5) (layer "F.Cu") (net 1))
 (segment (start 156.500123 70.999877) (end 155 72.5) (width 0.5) (layer "F.Cu") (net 1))
 (segment (start 182.5 59.76) (end 182.5 80) (width 0.5) (layer "F.Cu") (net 1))
 (segment (start 157.778811 64.721189) (end 156.500123 65.999877) (width 0.5) (layer "F.Cu") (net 1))
 (segment (start 163.811189 64.721189) (end 157.778811 64.721189) (width 0.5) (layer "F.Cu") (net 1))
 (segment (start 180.08 57.34) (end 182.5 59.76) (width 0.5) (layer "F.Cu") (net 1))
 (segment (start 153.335798 82.5) (end 150.5 82.5) (width 0.5) (layer "F.Cu") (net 1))
 (segment (start 132.5 82.5) (end 145.5 82.5) (width 0.5) (layer "F.Cu") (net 1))
 (segment (start 135.45 72.5) (end 142.5 72.5) (width 0.5) (layer "F.Cu") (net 1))
 (segment (start 132.725 69.775) (end 135.45 72.5) (width 0.5) (layer "F.Cu") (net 1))
 (segment (start 152.05 67.5) (end 149.55 65) (width 0.5) (layer "F.Cu") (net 1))
 (segment (start 145 72.5) (end 147.5 72.5) (width 0.5) (layer "F.Cu") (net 1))
 (segment (start 132.5 65.675) (end 132.5 70) (width 0.5) (layer "F.Cu") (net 1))
 (segment (start 182.5 80) (end 180 82.5) (width 0.5) (layer "F.Cu") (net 1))
 (segment (start 131.875 89.375) (end 143.625 89.375) (width 0.5) (layer "F.Cu") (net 1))
 (segment (start 160.835798 90) (end 153.335798 82.5) (width 0.5) (layer "F.Cu") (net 1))
 (segment (start 150.5 82.5) (end 147.75 85.25) (width 0.5) (layer "F.Cu") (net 1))
 (segment (start 177.5 90) (end 160.835798 90) (width 0.5) (layer "F.Cu") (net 1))
 (segment (start 145.5 82.5) (end 148 85) (width 0.5) (layer "F.Cu") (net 1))
 (segment (start 132.5 70) (end 132.5 82.5) (width 0.5) (layer "F.Cu") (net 1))
 (segment (start 147.75 85.25) (end 148 85) (width 0.5) (layer "F.Cu") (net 1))
 (segment (start 180 87.5) (end 177.5 90) (width 0.5) (layer "F.Cu") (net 1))
 (segment (start 132.5 65.675) (end 135 65.675) (width 0.5) (layer "F.Cu") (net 1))
 (segment (start 145.575 87.425) (end 147.75 85.25) (width 0.5) (layer "F.Cu") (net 1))
 (segment (start 180.16 57.34) (end 180.16 54.8) (width 0.5) (layer "F.Cu") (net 1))
 (segment (start 156.500123 65.999877) (end 156.500123 70.999877) (width 0.5) (layer "F.Cu") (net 1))
 (segment (start 155 72.5) (end 147.5 72.5) (width 0.5) (layer "F.Cu") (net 1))
 (segment (start 130 55) (end 131.684488 56.684488) (width 0.5) (layer "F.Cu") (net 5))
 (segment (start 155.362111 47.5) (end 137.5 47.5) (width 0.5) (layer "F.Cu") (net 5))
 (segment (start 135.95 60) (end 140 64.05) (width 0.5) (layer "F.Cu") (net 5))
 (segment (start 133.771 60) (end 135.95 60) (width 0.5) (layer "F.Cu") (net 5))
 (segment (start 131.684488 57.913488) (end 133.771 60) (width 0.5) (layer "F.Cu") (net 5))
 (segment (start 160 52.137889) (end 155.362111 47.5) (width 0.5) (layer "F.Cu") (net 5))
 (segment (start 137.5 47.5) (end 130 55) (width 0.5) (layer "F.Cu") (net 5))
 (segment (start 131.684488 56.684488) (end 131.684488 57.913488) (width 0.5) (layer "F.Cu") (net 5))
 (segment (start 160 60) (end 160 52.137889) (width 0.5) (layer "F.Cu") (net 5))
 (segment (start 140 64.05) (end 140 65) (width 0.5) (layer "F.Cu") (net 5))
 (segment (start 138.73 65.12314) (end 138.73 66.23) (width 0.5) (layer "F.Cu") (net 4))
 (segment (start 138.73 65) (end 138.73 65.12314) (width 0.2) (layer "F.Cu") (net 4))
 (segment (start 138.73 65) (end 138.73 65.225) (width 0.2) (layer "F.Cu") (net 4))
 (segment (start 140 67.5) (end 142.5 67.5) (width 0.5) (layer "F.Cu") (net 4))
 (segment (start 143.949 66.051) (end 144.0875 65.9125) (width 0.2) (layer "F.Cu") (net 4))
 (segment (start 138.73 66.23) (end 140 67.5) (width 0.5) (layer "F.Cu") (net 4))
 (segment (start 142.5 67.5) (end 143.949 66.051) (width 0.5) (layer "F.Cu") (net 4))
 (segment (start 160.675 62.5) (end 158.175 60) (width 0.5) (layer "F.Cu") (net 45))
 (segment (start 162.5 62.5) (end 160.675 62.5) (width 0.5) (layer "F.Cu") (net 45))
 (segment (start 169.92 57.34) (end 167.66 57.34) (width 0.5) (layer "F.Cu") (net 45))
 (segment (start 167.66 57.34) (end 162.5 62.5) (width 0.5) (layer "F.Cu") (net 45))
 (segment (start 162.5 75) (end 158.53 75) (width 0.2) (layer "F.Cu") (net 25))
 (segment (start 167.356 70.144) (end 167.356 70.286994) (width 0.2) (layer "F.Cu") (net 25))
 (segment (start 174.0424 68.5376) (end 168.9624 68.5376) (width 0.2) (layer "F.Cu") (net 25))
 (segment (start 180.16 62.42) (end 174.0424 68.5376) (width 0.2) (layer "F.Cu") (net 25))
 (segment (start 166.836994 70.806) (end 166.694 70.806) (width 0.2) (layer "F.Cu") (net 25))
 (segment (start 168.9624 68.5376) (end 167.356 70.144) (width 0.2) (layer "F.Cu") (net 25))
 (segment (start 167.356 70.286994) (end 166.836994 70.806) (width 0.2) (layer "F.Cu") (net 25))
 (segment (start 166.694 70.806) (end 162.5 75) (width 0.2) (layer "F.Cu") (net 25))
 (segment (start 158.53 69.92) (end 165.182994 69.92) (width 0.2) (layer "F.Cu") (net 23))
 (segment (start 169.105394 65.9976) (end 173.9624 65.9976) (width 0.2) (layer "F.Cu") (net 23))
 (segment (start 173.9624 65.9976) (end 180.08 59.88) (width 0.2) (layer "F.Cu") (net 23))
 (segment (start 165.182994 69.92) (end 169.105394 65.9976) (width 0.2) (layer "F.Cu") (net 23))
 (segment (start 169.105395 71.0776) (end 160.102995 80.08) (width 0.2) (layer "F.Cu") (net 26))
 (segment (start 160.102995 80.08) (end 158.53 80.08) (width 0.2) (layer "F.Cu") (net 26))
 (segment (start 180.16 64.96) (end 174.0424 71.0776) (width 0.2) (layer "F.Cu") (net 26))
 (segment (start 174.0424 71.0776) (end 169.105395 71.0776) (width 0.2) (layer "F.Cu") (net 26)))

